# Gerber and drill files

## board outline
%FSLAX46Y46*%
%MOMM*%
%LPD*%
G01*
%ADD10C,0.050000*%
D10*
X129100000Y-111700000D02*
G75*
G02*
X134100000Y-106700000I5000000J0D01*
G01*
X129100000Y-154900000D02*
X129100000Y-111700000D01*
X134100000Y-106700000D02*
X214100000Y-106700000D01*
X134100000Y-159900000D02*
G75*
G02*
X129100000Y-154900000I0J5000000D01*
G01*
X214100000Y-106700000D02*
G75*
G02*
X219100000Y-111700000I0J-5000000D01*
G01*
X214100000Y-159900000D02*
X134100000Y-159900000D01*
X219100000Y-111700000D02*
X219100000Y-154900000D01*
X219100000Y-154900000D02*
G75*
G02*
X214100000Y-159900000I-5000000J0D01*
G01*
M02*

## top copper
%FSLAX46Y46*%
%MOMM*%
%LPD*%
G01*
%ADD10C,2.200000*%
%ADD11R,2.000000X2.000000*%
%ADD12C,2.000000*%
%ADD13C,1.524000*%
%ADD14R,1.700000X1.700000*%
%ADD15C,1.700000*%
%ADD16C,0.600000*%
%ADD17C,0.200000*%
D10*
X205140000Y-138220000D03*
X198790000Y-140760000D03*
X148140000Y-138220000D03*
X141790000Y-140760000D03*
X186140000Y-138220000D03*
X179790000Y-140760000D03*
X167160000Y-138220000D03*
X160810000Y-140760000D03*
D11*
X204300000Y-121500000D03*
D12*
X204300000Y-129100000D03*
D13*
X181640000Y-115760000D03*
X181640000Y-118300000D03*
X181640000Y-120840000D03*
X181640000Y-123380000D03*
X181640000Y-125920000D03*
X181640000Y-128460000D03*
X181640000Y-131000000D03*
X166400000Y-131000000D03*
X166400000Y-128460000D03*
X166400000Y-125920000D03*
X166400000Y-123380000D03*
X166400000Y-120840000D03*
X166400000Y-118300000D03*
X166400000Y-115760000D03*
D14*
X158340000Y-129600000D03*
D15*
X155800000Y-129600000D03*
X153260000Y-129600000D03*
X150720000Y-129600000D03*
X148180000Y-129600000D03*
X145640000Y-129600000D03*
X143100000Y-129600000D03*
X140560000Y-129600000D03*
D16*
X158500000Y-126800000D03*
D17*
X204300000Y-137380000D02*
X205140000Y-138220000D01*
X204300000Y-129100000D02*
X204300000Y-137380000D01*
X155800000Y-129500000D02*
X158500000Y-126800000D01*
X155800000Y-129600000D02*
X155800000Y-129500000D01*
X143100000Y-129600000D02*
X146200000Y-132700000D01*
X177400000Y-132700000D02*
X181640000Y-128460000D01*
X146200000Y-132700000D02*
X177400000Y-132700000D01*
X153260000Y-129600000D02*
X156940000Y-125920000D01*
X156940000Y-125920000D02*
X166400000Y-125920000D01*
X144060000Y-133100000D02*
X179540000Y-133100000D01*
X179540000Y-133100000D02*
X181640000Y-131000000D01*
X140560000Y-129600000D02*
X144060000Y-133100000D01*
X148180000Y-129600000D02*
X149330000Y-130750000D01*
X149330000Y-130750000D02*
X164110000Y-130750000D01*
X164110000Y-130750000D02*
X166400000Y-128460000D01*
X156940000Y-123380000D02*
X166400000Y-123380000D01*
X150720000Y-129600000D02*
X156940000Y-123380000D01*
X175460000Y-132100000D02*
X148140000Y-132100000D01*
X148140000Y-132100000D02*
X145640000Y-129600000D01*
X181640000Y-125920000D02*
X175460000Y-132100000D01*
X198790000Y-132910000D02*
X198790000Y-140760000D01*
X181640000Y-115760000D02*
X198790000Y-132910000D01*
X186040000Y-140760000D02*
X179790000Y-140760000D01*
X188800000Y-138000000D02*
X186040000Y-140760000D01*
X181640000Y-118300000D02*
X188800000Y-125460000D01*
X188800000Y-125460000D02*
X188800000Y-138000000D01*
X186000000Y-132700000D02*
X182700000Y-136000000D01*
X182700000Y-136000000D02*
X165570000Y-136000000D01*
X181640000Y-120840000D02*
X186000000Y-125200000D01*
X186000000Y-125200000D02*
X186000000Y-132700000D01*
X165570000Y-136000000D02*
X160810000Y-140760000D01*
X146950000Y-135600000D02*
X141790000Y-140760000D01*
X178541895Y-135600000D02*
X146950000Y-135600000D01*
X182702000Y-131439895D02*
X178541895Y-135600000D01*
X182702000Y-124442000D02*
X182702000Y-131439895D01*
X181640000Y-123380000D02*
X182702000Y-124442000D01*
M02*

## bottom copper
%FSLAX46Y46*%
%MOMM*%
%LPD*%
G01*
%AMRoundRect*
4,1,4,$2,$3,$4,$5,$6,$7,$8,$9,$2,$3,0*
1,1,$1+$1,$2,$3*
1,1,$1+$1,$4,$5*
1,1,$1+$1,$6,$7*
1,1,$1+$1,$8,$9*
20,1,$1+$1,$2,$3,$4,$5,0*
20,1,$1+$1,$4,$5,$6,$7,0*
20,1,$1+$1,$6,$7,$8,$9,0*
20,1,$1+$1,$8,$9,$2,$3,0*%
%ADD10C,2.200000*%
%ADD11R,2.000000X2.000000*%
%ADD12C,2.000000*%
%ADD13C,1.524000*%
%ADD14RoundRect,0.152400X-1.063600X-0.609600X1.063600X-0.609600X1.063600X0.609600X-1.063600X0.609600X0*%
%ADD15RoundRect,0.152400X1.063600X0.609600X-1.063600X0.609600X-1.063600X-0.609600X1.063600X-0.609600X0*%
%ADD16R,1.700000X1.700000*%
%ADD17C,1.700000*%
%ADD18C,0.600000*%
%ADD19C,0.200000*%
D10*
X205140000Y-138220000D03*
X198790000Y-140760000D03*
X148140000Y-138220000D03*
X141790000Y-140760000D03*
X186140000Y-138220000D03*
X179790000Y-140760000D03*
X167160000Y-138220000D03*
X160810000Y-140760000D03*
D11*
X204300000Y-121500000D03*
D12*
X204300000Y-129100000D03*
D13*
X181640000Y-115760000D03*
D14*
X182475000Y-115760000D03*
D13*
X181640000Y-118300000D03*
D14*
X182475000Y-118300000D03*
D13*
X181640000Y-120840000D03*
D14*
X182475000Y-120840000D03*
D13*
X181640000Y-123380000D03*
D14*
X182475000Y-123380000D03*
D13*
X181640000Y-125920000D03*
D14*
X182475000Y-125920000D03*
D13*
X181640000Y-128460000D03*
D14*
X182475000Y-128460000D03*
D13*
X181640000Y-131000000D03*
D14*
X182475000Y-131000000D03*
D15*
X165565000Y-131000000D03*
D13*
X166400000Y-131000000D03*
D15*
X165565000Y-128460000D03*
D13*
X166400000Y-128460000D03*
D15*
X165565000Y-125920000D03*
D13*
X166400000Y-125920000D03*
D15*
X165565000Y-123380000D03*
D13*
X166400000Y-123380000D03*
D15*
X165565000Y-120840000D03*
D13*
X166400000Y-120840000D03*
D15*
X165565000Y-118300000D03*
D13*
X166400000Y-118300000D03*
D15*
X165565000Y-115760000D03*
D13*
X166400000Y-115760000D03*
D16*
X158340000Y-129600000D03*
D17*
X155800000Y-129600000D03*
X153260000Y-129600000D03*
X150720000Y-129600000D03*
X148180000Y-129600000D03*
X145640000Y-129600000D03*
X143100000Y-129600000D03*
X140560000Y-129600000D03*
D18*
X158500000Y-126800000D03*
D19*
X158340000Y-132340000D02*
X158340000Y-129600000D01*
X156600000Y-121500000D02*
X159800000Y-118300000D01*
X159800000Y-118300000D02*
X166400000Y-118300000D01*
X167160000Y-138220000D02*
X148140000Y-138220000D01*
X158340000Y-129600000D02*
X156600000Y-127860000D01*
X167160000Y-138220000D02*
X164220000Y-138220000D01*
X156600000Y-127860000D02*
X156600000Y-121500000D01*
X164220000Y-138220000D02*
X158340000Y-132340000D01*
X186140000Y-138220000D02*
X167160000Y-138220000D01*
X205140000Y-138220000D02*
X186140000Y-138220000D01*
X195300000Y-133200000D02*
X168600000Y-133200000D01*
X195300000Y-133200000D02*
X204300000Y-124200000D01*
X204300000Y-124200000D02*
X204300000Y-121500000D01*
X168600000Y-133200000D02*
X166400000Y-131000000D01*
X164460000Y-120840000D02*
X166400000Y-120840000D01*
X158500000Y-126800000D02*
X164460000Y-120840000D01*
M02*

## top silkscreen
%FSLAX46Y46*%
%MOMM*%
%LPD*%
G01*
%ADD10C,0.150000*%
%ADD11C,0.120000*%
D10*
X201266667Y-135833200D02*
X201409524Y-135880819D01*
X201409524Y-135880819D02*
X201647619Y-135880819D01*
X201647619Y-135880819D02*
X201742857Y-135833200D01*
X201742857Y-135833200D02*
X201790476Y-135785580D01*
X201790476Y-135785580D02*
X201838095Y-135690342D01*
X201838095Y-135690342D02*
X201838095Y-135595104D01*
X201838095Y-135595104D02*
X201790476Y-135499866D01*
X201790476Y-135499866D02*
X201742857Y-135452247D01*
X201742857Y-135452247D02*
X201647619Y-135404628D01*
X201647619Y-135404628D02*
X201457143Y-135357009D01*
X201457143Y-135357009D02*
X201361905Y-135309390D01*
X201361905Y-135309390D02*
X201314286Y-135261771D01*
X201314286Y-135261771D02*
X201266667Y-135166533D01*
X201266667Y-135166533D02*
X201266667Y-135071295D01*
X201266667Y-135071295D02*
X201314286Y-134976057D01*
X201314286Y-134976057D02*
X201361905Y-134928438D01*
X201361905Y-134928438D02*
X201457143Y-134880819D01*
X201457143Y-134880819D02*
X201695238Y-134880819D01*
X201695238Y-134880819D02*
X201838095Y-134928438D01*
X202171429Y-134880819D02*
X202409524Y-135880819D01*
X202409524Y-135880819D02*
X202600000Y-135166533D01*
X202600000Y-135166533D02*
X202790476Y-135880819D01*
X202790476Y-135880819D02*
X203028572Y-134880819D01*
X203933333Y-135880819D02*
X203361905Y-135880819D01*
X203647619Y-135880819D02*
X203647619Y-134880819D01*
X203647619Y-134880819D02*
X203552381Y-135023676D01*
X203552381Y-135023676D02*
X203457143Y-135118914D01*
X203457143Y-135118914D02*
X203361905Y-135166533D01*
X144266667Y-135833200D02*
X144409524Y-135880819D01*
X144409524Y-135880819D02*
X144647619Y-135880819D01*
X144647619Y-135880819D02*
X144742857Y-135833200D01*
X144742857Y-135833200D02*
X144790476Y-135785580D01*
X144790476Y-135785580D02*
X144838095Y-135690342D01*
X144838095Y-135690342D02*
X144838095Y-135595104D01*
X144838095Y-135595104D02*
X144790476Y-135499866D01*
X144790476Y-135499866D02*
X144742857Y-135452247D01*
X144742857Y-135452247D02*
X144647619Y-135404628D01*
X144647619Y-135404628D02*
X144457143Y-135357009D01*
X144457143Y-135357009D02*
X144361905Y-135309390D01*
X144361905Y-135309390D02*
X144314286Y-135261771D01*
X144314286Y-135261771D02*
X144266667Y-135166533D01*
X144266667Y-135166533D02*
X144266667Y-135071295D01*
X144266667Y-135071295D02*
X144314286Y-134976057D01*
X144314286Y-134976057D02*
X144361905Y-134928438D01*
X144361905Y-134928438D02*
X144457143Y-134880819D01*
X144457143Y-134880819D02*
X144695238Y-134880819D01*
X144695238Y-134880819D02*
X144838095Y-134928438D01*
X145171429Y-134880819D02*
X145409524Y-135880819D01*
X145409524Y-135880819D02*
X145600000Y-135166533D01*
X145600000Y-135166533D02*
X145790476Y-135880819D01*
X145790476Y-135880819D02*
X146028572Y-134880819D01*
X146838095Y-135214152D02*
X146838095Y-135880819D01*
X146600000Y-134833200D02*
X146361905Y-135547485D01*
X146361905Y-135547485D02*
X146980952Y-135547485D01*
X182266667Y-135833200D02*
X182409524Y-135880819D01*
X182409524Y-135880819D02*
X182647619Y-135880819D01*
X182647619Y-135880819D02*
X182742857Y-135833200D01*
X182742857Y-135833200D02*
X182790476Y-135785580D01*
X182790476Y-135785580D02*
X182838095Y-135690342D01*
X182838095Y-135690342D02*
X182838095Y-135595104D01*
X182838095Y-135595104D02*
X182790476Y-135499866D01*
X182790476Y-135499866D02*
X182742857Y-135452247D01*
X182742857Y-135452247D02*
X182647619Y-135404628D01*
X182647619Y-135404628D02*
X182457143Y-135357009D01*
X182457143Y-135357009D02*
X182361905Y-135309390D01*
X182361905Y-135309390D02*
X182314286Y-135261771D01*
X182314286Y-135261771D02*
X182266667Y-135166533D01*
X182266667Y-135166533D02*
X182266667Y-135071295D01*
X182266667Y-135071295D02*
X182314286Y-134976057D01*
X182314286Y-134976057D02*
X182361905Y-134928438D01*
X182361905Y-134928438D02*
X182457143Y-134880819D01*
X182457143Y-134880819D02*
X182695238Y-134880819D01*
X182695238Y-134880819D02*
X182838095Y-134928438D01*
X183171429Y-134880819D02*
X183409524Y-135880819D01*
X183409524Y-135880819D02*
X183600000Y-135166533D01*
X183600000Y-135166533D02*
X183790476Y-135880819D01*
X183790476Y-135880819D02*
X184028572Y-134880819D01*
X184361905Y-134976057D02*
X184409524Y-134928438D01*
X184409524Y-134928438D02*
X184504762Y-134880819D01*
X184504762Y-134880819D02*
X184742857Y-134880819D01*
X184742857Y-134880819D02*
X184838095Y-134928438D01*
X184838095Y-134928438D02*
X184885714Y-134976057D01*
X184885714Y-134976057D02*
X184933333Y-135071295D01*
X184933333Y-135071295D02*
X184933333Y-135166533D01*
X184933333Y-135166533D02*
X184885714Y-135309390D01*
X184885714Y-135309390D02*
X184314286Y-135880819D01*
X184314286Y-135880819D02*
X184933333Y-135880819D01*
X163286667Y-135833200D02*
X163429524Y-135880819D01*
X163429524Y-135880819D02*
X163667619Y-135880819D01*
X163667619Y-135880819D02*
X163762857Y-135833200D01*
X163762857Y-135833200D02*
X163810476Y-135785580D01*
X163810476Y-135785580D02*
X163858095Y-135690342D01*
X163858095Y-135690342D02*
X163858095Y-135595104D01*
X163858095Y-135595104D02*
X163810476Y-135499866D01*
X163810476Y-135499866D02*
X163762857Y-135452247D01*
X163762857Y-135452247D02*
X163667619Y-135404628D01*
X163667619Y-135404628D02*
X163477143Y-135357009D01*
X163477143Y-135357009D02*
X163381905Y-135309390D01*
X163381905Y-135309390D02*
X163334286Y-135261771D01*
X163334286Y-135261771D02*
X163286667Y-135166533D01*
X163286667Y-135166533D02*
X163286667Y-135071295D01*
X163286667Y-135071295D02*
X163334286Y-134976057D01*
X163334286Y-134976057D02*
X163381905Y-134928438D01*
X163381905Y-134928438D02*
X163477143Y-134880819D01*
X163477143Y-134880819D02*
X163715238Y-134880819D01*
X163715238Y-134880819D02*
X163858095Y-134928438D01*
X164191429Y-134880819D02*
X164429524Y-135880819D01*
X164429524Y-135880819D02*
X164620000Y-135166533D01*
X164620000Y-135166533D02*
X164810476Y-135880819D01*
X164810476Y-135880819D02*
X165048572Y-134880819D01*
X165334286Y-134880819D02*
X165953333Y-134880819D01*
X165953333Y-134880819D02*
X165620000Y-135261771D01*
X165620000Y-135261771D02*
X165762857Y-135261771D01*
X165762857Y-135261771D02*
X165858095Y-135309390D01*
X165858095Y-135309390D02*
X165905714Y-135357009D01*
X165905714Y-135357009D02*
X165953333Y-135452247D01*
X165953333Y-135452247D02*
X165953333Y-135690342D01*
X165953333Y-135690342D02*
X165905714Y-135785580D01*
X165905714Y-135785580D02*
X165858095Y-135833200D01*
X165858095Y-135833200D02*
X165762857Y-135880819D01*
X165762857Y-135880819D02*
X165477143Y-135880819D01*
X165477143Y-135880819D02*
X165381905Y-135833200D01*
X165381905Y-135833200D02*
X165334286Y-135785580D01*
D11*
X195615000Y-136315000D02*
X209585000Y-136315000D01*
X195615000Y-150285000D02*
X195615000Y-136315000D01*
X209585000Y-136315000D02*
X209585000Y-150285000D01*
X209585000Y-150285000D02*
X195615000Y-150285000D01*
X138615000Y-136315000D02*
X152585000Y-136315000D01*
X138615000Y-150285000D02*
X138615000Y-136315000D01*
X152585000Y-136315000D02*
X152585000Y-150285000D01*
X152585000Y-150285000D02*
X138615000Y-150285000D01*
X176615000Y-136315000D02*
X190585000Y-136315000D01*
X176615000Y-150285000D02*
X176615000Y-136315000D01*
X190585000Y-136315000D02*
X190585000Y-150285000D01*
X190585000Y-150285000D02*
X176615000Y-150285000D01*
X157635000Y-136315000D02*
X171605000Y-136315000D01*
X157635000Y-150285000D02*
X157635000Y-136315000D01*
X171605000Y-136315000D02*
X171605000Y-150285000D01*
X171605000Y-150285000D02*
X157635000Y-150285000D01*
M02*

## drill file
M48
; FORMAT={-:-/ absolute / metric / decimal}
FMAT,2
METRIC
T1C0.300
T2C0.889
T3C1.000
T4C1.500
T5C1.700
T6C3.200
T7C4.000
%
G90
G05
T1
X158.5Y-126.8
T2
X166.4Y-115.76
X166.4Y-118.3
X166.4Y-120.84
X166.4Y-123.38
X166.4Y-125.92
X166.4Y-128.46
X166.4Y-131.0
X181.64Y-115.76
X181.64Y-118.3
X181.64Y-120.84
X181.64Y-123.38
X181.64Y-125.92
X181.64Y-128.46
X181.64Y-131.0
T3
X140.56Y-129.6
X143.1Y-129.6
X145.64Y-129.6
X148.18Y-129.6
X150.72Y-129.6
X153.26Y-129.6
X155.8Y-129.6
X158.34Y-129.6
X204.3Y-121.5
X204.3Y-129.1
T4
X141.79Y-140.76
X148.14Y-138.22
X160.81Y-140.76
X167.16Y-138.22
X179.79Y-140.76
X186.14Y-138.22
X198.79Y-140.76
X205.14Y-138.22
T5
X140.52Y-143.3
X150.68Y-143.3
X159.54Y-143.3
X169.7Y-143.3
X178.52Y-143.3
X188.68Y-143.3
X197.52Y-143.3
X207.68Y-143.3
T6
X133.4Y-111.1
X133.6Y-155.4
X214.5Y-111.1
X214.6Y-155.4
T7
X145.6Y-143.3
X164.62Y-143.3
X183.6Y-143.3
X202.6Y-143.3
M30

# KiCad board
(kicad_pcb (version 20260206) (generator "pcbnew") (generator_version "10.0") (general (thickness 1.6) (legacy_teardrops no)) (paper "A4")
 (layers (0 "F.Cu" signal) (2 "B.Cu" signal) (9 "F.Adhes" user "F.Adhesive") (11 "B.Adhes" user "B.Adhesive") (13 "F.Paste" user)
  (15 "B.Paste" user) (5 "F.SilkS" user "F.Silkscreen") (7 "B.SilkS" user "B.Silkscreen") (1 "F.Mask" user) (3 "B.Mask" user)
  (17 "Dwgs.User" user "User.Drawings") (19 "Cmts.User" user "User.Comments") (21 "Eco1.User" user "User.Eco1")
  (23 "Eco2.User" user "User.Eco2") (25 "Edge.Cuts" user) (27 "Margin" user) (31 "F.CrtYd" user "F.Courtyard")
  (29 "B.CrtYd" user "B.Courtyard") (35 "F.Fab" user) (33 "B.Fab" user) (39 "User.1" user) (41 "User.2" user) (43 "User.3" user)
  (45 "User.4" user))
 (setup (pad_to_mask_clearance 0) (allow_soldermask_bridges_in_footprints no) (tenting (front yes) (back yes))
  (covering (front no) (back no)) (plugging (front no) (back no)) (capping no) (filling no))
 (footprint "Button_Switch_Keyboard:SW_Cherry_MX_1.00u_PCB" (layer "F.Cu") (at 205.14 138.22)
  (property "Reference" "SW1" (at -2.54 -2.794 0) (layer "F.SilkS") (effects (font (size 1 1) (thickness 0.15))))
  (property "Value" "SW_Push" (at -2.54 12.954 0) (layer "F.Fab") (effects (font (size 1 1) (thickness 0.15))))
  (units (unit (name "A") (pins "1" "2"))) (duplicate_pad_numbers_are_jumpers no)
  (fp_line (start -9.525 -1.905) (end 4.445 -1.905) (stroke (width 0.12) (type solid)) (layer "F.SilkS"))
  (fp_line (start -9.525 12.065) (end -9.525 -1.905) (stroke (width 0.12) (type solid)) (layer "F.SilkS"))
  (fp_line (start 4.445 -1.905) (end 4.445 12.065) (stroke (width 0.12) (type solid)) (layer "F.SilkS"))
  (fp_line (start 4.445 12.065) (end -9.525 12.065) (stroke (width 0.12) (type solid)) (layer "F.SilkS"))
  (pad "" np_thru_hole circle (at -7.62 5.08) (size 1.7 1.7) (drill 1.7) (layers "*.Cu" "*.Mask"))
  (pad "" np_thru_hole circle (at -2.54 5.08) (size 4 4) (drill 4) (layers "*.Cu" "*.Mask"))
  (pad "" np_thru_hole circle (at 2.54 5.08) (size 1.7 1.7) (drill 1.7) (layers "*.Cu" "*.Mask"))
  (pad "1" thru_hole circle (at 0 0) (size 2.2 2.2) (drill 1.5) (layers "*.Cu" "*.Mask") (remove_unused_layers no) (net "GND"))
  (pad "2" thru_hole circle (at -6.35 2.54) (size 2.2 2.2) (drill 1.5) (layers "*.Cu" "*.Mask") (remove_unused_layers no)
   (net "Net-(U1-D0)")))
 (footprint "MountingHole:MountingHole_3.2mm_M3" (layer "F.Cu") (at 133.4 111.1)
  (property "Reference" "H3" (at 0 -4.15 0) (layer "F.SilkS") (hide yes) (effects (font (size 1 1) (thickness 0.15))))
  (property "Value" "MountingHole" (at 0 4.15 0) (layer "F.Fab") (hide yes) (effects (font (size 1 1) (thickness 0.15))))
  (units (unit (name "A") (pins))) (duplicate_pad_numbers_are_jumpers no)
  (pad "" np_thru_hole circle (at 0 0) (size 3.2 3.2) (drill 3.2) (layers "*.Cu" "*.Mask")))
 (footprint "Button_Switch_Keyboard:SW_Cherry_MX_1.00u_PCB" (layer "F.Cu") (at 148.14 138.22)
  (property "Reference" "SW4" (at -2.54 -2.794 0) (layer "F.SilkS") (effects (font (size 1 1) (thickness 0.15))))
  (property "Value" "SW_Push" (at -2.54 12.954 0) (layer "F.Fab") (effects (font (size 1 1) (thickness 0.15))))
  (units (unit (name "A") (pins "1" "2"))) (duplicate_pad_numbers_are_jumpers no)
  (fp_line (start -9.525 -1.905) (end 4.445 -1.905) (stroke (width 0.12) (type solid)) (layer "F.SilkS"))
  (fp_line (start -9.525 12.065) (end -9.525 -1.905) (stroke (width 0.12) (type solid)) (layer "F.SilkS"))
  (fp_line (start 4.445 -1.905) (end 4.445 12.065) (stroke (width 0.12) (type solid)) (layer "F.SilkS"))
  (fp_line (start 4.445 12.065) (end -9.525 12.065) (stroke (width 0.12) (type solid)) (layer "F.SilkS"))
  (pad "" np_thru_hole circle (at -7.62 5.08) (size 1.7 1.7) (drill 1.7) (layers "*.Cu" "*.Mask"))
  (pad "" np_thru_hole circle (at -2.54 5.08) (size 4 4) (drill 4) (layers "*.Cu" "*.Mask"))
  (pad "" np_thru_hole circle (at 2.54 5.08) (size 1.7 1.7) (drill 1.7) (layers "*.Cu" "*.Mask"))
  (pad "1" thru_hole circle (at 0 0) (size 2.2 2.2) (drill 1.5) (layers "*.Cu" "*.Mask") (remove_unused_layers no) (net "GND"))
  (pad "2" thru_hole circle (at -6.35 2.54) (size 2.2 2.2) (drill 1.5) (layers "*.Cu" "*.Mask") (remove_unused_layers no)
   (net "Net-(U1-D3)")))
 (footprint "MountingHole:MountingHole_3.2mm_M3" (layer "F.Cu") (at 133.6 155.4)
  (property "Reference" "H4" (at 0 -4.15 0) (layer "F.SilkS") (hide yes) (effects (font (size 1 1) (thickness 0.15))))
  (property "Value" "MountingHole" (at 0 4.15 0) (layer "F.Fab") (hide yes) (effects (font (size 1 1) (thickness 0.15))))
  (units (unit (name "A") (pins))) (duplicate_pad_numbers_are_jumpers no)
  (pad "" np_thru_hole circle (at 0 0) (size 3.2 3.2) (drill 3.2) (layers "*.Cu" "*.Mask")))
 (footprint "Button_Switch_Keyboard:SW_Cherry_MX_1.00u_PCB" (layer "F.Cu") (at 186.14 138.22)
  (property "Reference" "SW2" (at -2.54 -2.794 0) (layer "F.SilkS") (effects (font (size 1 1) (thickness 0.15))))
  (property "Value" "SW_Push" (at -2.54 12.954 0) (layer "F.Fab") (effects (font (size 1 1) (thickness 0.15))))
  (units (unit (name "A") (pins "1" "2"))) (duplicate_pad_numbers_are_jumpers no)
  (fp_line (start -9.525 -1.905) (end 4.445 -1.905) (stroke (width 0.12) (type solid)) (layer "F.SilkS"))
  (fp_line (start -9.525 12.065) (end -9.525 -1.905) (stroke (width 0.12) (type solid)) (layer "F.SilkS"))
  (fp_line (start 4.445 -1.905) (end 4.445 12.065) (stroke (width 0.12) (type solid)) (layer "F.SilkS"))
  (fp_line (start 4.445 12.065) (end -9.525 12.065) (stroke (width 0.12) (type solid)) (layer "F.SilkS"))
  (pad "" np_thru_hole circle (at -7.62 5.08) (size 1.7 1.7) (drill 1.7) (layers "*.Cu" "*.Mask"))
  (pad "" np_thru_hole circle (at -2.54 5.08) (size 4 4) (drill 4) (layers "*.Cu" "*.Mask"))
  (pad "" np_thru_hole circle (at 2.54 5.08) (size 1.7 1.7) (drill 1.7) (layers "*.Cu" "*.Mask"))
  (pad "1" thru_hole circle (at 0 0) (size 2.2 2.2) (drill 1.5) (layers "*.Cu" "*.Mask") (remove_unused_layers no) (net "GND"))
  (pad "2" thru_hole circle (at -6.35 2.54) (size 2.2 2.2) (drill 1.5) (layers "*.Cu" "*.Mask") (remove_unused_layers no)
   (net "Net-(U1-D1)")))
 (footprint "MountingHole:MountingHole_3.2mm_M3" (layer "F.Cu") (at 214.5 111.1)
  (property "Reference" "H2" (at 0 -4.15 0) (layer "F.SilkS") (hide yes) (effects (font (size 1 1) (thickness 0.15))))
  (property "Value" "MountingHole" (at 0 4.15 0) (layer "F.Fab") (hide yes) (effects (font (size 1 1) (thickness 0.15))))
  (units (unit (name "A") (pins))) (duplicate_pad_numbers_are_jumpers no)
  (pad "" np_thru_hole circle (at 0 0) (size 3.2 3.2) (drill 3.2) (layers "*.Cu" "*.Mask")))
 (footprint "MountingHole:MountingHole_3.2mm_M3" (layer "F.Cu") (at 214.6 155.4)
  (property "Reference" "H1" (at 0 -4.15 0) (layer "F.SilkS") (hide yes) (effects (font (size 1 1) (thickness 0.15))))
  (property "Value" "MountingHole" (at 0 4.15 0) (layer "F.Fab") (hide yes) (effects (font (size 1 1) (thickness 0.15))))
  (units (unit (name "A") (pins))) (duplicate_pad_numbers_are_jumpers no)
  (pad "" np_thru_hole circle (at 0 0) (size 3.2 3.2) (drill 3.2) (layers "*.Cu" "*.Mask")))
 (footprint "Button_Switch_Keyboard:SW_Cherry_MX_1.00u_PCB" (layer "F.Cu") (at 167.16 138.22)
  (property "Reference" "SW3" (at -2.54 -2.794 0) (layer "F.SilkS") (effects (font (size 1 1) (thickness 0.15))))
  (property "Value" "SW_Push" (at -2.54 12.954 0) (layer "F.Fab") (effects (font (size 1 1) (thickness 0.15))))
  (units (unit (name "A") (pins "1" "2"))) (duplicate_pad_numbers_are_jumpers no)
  (fp_line (start -9.525 -1.905) (end 4.445 -1.905) (stroke (width 0.12) (type solid)) (layer "F.SilkS"))
  (fp_line (start -9.525 12.065) (end -9.525 -1.905) (stroke (width 0.12) (type solid)) (layer "F.SilkS"))
  (fp_line (start 4.445 -1.905) (end 4.445 12.065) (stroke (width 0.12) (type solid)) (layer "F.SilkS"))
  (fp_line (start 4.445 12.065) (end -9.525 12.065) (stroke (width 0.12) (type solid)) (layer "F.SilkS"))
  (pad "" np_thru_hole circle (at -7.62 5.08) (size 1.7 1.7) (drill 1.7) (layers "*.Cu" "*.Mask"))
  (pad "" np_thru_hole circle (at -2.54 5.08) (size 4 4) (drill 4) (layers "*.Cu" "*.Mask"))
  (pad "" np_thru_hole circle (at 2.54 5.08) (size 1.7 1.7) (drill 1.7) (layers "*.Cu" "*.Mask"))
  (pad "1" thru_hole circle (at 0 0) (size 2.2 2.2) (drill 1.5) (layers "*.Cu" "*.Mask") (remove_unused_layers no) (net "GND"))
  (pad "2" thru_hole circle (at -6.35 2.54) (size 2.2 2.2) (drill 1.5) (layers "*.Cu" "*.Mask") (remove_unused_layers no)
   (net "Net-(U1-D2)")))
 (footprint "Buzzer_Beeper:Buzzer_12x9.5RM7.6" (layer "B.Cu") (at 204.3 121.5 -90)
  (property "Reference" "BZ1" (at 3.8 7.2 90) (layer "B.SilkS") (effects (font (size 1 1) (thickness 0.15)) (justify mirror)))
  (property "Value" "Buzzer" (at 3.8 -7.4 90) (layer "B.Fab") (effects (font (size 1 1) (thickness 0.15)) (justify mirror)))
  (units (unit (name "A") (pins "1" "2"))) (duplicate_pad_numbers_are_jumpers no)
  (pad "1" thru_hole rect (at 0 0 270) (size 2 2) (drill 1) (layers "*.Cu" "*.Mask") (remove_unused_layers no) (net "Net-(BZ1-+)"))
  (pad "2" thru_hole circle (at 7.6 0 270) (size 2 2) (drill 1) (layers "*.Cu" "*.Mask") (remove_unused_layers no) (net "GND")))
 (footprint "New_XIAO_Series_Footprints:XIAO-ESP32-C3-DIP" (layer "B.Cu") (at 174.02 123.38 90)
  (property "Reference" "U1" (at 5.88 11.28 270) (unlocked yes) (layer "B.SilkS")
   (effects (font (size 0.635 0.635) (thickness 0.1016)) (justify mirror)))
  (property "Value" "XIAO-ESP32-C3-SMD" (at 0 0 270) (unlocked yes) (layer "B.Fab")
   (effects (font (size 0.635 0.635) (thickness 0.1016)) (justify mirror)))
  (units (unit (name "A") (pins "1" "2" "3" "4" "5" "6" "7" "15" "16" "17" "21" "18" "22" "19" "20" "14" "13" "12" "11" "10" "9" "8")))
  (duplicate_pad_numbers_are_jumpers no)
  (pad "1" thru_hole circle (at 7.62 7.62) (size 1.524 1.524) (drill 0.889) (layers "*.Cu" "*.Mask") (remove_unused_layers no)
   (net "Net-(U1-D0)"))
  (pad "1" smd roundrect (at 7.62 8.455) (size 2.432 1.524) (layers "B.Cu" "B.Mask") (roundrect_rratio 0.1) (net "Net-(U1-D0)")
   (thermal_bridge_angle 45))
  (pad "2" thru_hole circle (at 5.08 7.62) (size 1.524 1.524) (drill 0.889) (layers "*.Cu" "*.Mask") (remove_unused_layers no)
   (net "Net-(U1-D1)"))
  (pad "2" smd roundrect (at 5.08 8.455) (size 2.432 1.524) (layers "B.Cu" "B.Mask") (roundrect_rratio 0.1) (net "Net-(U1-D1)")
   (thermal_bridge_angle 45))
  (pad "3" thru_hole circle (at 2.54 7.62) (size 1.524 1.524) (drill 0.889) (layers "*.Cu" "*.Mask") (remove_unused_layers no)
   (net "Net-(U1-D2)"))
  (pad "3" smd roundrect (at 2.54 8.455) (size 2.432 1.524) (layers "B.Cu" "B.Mask") (roundrect_rratio 0.1) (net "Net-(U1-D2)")
   (thermal_bridge_angle 45))
  (pad "4" thru_hole circle (at 0 7.62) (size 1.524 1.524) (drill 0.889) (layers "*.Cu" "*.Mask") (remove_unused_layers no)
   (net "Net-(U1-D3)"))
  (pad "4" smd roundrect (at 0 8.455) (size 2.432 1.524) (layers "B.Cu" "B.Mask") (roundrect_rratio 0.1) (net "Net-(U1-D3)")
   (thermal_bridge_angle 45))
  (pad "5" thru_hole circle (at -2.54 7.62) (size 1.524 1.524) (drill 0.889) (layers "*.Cu" "*.Mask") (remove_unused_layers no) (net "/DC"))
  (pad "5" smd roundrect (at -2.54 8.455) (size 2.432 1.524) (layers "B.Cu" "B.Mask") (roundrect_rratio 0.1) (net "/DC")
   (thermal_bridge_angle 45))
  (pad "6" thru_hole circle (at -5.08 7.62) (size 1.524 1.524) (drill 0.889) (layers "*.Cu" "*.Mask") (remove_unused_layers no) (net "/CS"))
  (pad "6" smd roundrect (at -5.08 8.455) (size 2.432 1.524) (layers "B.Cu" "B.Mask") (roundrect_rratio 0.1) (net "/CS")
   (thermal_bridge_angle 45))
  (pad "7" thru_hole circle (at -7.62 7.62) (size 1.524 1.524) (drill 0.889) (layers "*.Cu" "*.Mask") (remove_unused_layers no) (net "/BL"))
  (pad "7" smd roundrect (at -7.62 8.455) (size 2.432 1.524) (layers "B.Cu" "B.Mask") (roundrect_rratio 0.1) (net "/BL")
   (thermal_bridge_angle 45))
  (pad "8" smd roundrect (at -7.62 -8.455 180) (size 2.432 1.524) (layers "B.Cu" "B.Mask") (roundrect_rratio 0.1) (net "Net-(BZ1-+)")
   (thermal_bridge_angle 45))
  (pad "8" thru_hole circle (at -7.62 -7.62 180) (size 1.524 1.524) (drill 0.889) (layers "*.Cu" "*.Mask") (remove_unused_layers no)
   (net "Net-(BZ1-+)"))
  (pad "9" smd roundrect (at -5.08 -8.455 180) (size 2.432 1.524) (layers "B.Cu" "B.Mask") (roundrect_rratio 0.1) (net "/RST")
   (thermal_bridge_angle 45))
  (pad "9" thru_hole circle (at -5.08 -7.62 180) (size 1.524 1.524) (drill 0.889) (layers "*.Cu" "*.Mask") (remove_unused_layers no)
   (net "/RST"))
  (pad "10" smd roundrect (at -2.54 -8.455 180) (size 2.432 1.524) (layers "B.Cu" "B.Mask") (roundrect_rratio 0.1) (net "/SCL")
   (thermal_bridge_angle 45))
  (pad "10" thru_hole circle (at -2.54 -7.62 180) (size 1.524 1.524) (drill 0.889) (layers "*.Cu" "*.Mask") (remove_unused_layers no)
   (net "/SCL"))
  (pad "11" smd roundrect (at 0 -8.455 180) (size 2.432 1.524) (layers "B.Cu" "B.Mask") (roundrect_rratio 0.1) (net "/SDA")
   (thermal_bridge_angle 45))
  (pad "11" thru_hole circle (at 0 -7.62 180) (size 1.524 1.524) (drill 0.889) (layers "*.Cu" "*.Mask") (remove_unused_layers no)
   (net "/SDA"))
  (pad "12" smd roundrect (at 2.54 -8.455 180) (size 2.432 1.524) (layers "B.Cu" "B.Mask") (roundrect_rratio 0.1) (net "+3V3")
   (thermal_bridge_angle 45))
  (pad "12" thru_hole circle (at 2.54 -7.62 180) (size 1.524 1.524) (drill 0.889) (layers "*.Cu" "*.Mask") (remove_unused_layers no)
   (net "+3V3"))
  (pad "13" smd roundrect (at 5.08 -8.455 180) (size 2.432 1.524) (layers "B.Cu" "B.Mask") (roundrect_rratio 0.1) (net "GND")
   (thermal_bridge_angle 45))
  (pad "13" thru_hole circle (at 5.08 -7.62 180) (size 1.524 1.524) (drill 0.889) (layers "*.Cu" "*.Mask") (remove_unused_layers no)
   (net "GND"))
  (pad "14" smd roundrect (at 7.62 -8.455 180) (size 2.432 1.524) (layers "B.Cu" "B.Mask") (roundrect_rratio 0.1)
   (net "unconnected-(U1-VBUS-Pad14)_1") (thermal_bridge_angle 45))
  (pad "14" thru_hole circle (at 7.62 -7.62 180) (size 1.524 1.524) (drill 0.889) (layers "*.Cu" "*.Mask") (remove_unused_layers no)
   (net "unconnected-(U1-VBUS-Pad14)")))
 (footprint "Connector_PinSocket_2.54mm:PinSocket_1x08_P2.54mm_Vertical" (layer "B.Cu") (at 158.34 129.6 90)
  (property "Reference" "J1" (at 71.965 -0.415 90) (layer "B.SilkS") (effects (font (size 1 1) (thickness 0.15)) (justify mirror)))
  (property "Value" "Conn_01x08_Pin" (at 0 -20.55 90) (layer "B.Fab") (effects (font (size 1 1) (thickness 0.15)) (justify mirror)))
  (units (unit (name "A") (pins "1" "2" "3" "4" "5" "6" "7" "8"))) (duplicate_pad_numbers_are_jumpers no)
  (pad "1" thru_hole rect (at 0 0 90) (size 1.7 1.7) (drill 1) (layers "*.Cu" "*.Mask") (remove_unused_layers no) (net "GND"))
  (pad "2" thru_hole circle (at 0 -2.54 90) (size 1.7 1.7) (drill 1) (layers "*.Cu" "*.Mask") (remove_unused_layers no) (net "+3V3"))
  (pad "3" thru_hole circle (at 0 -5.08 90) (size 1.7 1.7) (drill 1) (layers "*.Cu" "*.Mask") (remove_unused_layers no) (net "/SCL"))
  (pad "4" thru_hole circle (at 0 -7.62 90) (size 1.7 1.7) (drill 1) (layers "*.Cu" "*.Mask") (remove_unused_layers no) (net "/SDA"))
  (pad "5" thru_hole circle (at 0 -10.16 90) (size 1.7 1.7) (drill 1) (layers "*.Cu" "*.Mask") (remove_unused_layers no) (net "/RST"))
  (pad "6" thru_hole circle (at 0 -12.7 90) (size 1.7 1.7) (drill 1) (layers "*.Cu" "*.Mask") (remove_unused_layers no) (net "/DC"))
  (pad "7" thru_hole circle (at 0 -15.24 90) (size 1.7 1.7) (drill 1) (layers "*.Cu" "*.Mask") (remove_unused_layers no) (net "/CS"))
  (pad "8" thru_hole circle (at 0 -17.78 90) (size 1.7 1.7) (drill 1) (layers "*.Cu" "*.Mask") (remove_unused_layers no) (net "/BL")))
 (gr_arc (start 129.1 111.7) (mid 130.564466 108.164466) (end 134.1 106.7) (stroke (width 0.05) (type default)) (layer "Edge.Cuts"))
 (gr_line (start 129.1 154.9) (end 129.1 111.7) (stroke (width 0.05) (type default)) (layer "Edge.Cuts"))
 (gr_line (start 134.1 106.7) (end 214.1 106.7) (stroke (width 0.05) (type default)) (layer "Edge.Cuts"))
 (gr_arc (start 134.1 159.9) (mid 130.564466 158.435534) (end 129.1 154.9) (stroke (width 0.05) (type default)) (layer "Edge.Cuts"))
 (gr_arc (start 214.1 106.7) (mid 217.635534 108.164466) (end 219.1 111.7) (stroke (width 0.05) (type default)) (layer "Edge.Cuts"))
 (gr_line (start 214.1 159.9) (end 134.1 159.9) (stroke (width 0.05) (type default)) (layer "Edge.Cuts"))
 (gr_line (start 219.1 111.7) (end 219.1 154.9) (stroke (width 0.05) (type default)) (layer "Edge.Cuts"))
 (gr_arc (start 219.1 154.9) (mid 217.635534 158.435534) (end 214.1 159.9) (stroke (width 0.05) (type default)) (layer "Edge.Cuts"))
 (segment (start 204.3 137.38) (end 205.14 138.22) (width 0.2) (layer "F.Cu") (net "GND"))
 (segment (start 204.3 129.1) (end 204.3 137.38) (width 0.2) (layer "F.Cu") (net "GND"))
 (segment (start 158.34 132.34) (end 158.34 129.6) (width 0.2) (layer "B.Cu") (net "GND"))
 (segment (start 156.6 121.5) (end 159.8 118.3) (width 0.2) (layer "B.Cu") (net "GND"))
 (segment (start 159.8 118.3) (end 166.4 118.3) (width 0.2) (layer "B.Cu") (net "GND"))
 (segment (start 167.16 138.22) (end 148.14 138.22) (width 0.2) (layer "B.Cu") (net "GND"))
 (segment (start 158.34 129.6) (end 156.6 127.86) (width 0.2) (layer "B.Cu") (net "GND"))
 (segment (start 167.16 138.22) (end 164.22 138.22) (width 0.2) (layer "B.Cu") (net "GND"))
 (segment (start 156.6 127.86) (end 156.6 121.5) (width 0.2) (layer "B.Cu") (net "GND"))
 (segment (start 164.22 138.22) (end 158.34 132.34) (width 0.2) (layer "B.Cu") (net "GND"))
 (segment (start 186.14 138.22) (end 167.16 138.22) (width 0.2) (layer "B.Cu") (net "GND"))
 (segment (start 205.14 138.22) (end 186.14 138.22) (width 0.2) (layer "B.Cu") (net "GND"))
 (segment (start 195.3 133.2) (end 168.6 133.2) (width 0.2) (layer "B.Cu") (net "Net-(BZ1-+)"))
 (segment (start 195.3 133.2) (end 204.3 124.2) (width 0.2) (layer "B.Cu") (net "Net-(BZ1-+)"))
 (segment (start 204.3 124.2) (end 204.3 121.5) (width 0.2) (layer "B.Cu") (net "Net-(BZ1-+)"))
 (segment (start 168.6 133.2) (end 166.4 131) (width 0.2) (layer "B.Cu") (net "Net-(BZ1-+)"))
 (segment (start 155.8 129.5) (end 158.5 126.8) (width 0.2) (layer "F.Cu") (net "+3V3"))
 (segment (start 155.8 129.6) (end 155.8 129.5) (width 0.2) (layer "F.Cu") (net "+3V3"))
 (via (at 158.5 126.8) (size 0.6) (drill 0.3) (layers "F.Cu" "B.Cu") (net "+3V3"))
 (segment (start 164.46 120.84) (end 166.4 120.84) (width 0.2) (layer "B.Cu") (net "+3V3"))
 (segment (start 158.5 126.8) (end 164.46 120.84) (width 0.2) (layer "B.Cu") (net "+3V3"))
 (segment (start 143.1 129.6) (end 146.2 132.7) (width 0.2) (layer "F.Cu") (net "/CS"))
 (segment (start 177.4 132.7) (end 181.64 128.46) (width 0.2) (layer "F.Cu") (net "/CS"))
 (segment (start 146.2 132.7) (end 177.4 132.7) (width 0.2) (layer "F.Cu") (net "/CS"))
 (segment (start 153.26 129.6) (end 156.94 125.92) (width 0.2) (layer "F.Cu") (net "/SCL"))
 (segment (start 156.94 125.92) (end 166.4 125.92) (width 0.2) (layer "F.Cu") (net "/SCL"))
 (segment (start 144.06 133.1) (end 179.54 133.1) (width 0.2) (layer "F.Cu") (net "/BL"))
 (segment (start 179.54 133.1) (end 181.64 131) (width 0.2) (layer "F.Cu") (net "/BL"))
 (segment (start 140.56 129.6) (end 144.06 133.1) (width 0.2) (layer "F.Cu") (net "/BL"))
 (segment (start 148.18 129.6) (end 149.33 130.75) (width 0.2) (layer "F.Cu") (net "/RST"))
 (segment (start 149.33 130.75) (end 164.11 130.75) (width 0.2) (layer "F.Cu") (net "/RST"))
 (segment (start 164.11 130.75) (end 166.4 128.46) (width 0.2) (layer "F.Cu") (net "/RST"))
 (segment (start 156.94 123.38) (end 166.4 123.38) (width 0.2) (layer "F.Cu") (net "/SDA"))
 (segment (start 150.72 129.6) (end 156.94 123.38) (width 0.2) (layer "F.Cu") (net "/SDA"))
 (segment (start 175.46 132.1) (end 148.14 132.1) (width 0.2) (layer "F.Cu") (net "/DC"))
 (segment (start 148.14 132.1) (end 145.64 129.6) (width 0.2) (layer "F.Cu") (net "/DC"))
 (segment (start 181.64 125.92) (end 175.46 132.1) (width 0.2) (layer "F.Cu") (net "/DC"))
 (segment (start 198.79 132.91) (end 198.79 140.76) (width 0.2) (layer "F.Cu") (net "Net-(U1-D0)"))
 (segment (start 181.64 115.76) (end 198.79 132.91) (width 0.2) (layer "F.Cu") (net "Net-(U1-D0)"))
 (segment (start 186.04 140.76) (end 179.79 140.76) (width 0.2) (layer "F.Cu") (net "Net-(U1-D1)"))
 (segment (start 188.8 138) (end 186.04 140.76) (width 0.2) (layer "F.Cu") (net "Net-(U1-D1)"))
 (segment (start 181.64 118.3) (end 188.8 125.46) (width 0.2) (layer "F.Cu") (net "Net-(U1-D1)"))
 (segment (start 188.8 125.46) (end 188.8 138) (width 0.2) (layer "F.Cu") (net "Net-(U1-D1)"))
 (segment (start 186 132.7) (end 182.7 136) (width 0.2) (layer "F.Cu") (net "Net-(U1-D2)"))
 (segment (start 182.7 136) (end 165.57 136) (width 0.2) (layer "F.Cu") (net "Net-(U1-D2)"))
 (segment (start 181.64 120.84) (end 186 125.2) (width 0.2) (layer "F.Cu") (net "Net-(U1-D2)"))
 (segment (start 186 125.2) (end 186 132.7) (width 0.2) (layer "F.Cu") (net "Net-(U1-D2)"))
 (segment (start 165.57 136) (end 160.81 140.76) (width 0.2) (layer "F.Cu") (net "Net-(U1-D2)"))
 (segment (start 146.95 135.6) (end 141.79 140.76) (width 0.2) (layer "F.Cu") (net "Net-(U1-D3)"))
 (segment (start 178.541895 135.6) (end 146.95 135.6) (width 0.2) (layer "F.Cu") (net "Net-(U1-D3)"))
 (segment (start 182.702 131.439895) (end 178.541895 135.6) (width 0.2) (layer "F.Cu") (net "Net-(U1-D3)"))
 (segment (start 182.702 124.442) (end 182.702 131.439895) (width 0.2) (layer "F.Cu") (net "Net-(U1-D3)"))
 (segment (start 181.64 123.38) (end 182.702 124.442) (width 0.2) (layer "F.Cu") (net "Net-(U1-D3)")))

